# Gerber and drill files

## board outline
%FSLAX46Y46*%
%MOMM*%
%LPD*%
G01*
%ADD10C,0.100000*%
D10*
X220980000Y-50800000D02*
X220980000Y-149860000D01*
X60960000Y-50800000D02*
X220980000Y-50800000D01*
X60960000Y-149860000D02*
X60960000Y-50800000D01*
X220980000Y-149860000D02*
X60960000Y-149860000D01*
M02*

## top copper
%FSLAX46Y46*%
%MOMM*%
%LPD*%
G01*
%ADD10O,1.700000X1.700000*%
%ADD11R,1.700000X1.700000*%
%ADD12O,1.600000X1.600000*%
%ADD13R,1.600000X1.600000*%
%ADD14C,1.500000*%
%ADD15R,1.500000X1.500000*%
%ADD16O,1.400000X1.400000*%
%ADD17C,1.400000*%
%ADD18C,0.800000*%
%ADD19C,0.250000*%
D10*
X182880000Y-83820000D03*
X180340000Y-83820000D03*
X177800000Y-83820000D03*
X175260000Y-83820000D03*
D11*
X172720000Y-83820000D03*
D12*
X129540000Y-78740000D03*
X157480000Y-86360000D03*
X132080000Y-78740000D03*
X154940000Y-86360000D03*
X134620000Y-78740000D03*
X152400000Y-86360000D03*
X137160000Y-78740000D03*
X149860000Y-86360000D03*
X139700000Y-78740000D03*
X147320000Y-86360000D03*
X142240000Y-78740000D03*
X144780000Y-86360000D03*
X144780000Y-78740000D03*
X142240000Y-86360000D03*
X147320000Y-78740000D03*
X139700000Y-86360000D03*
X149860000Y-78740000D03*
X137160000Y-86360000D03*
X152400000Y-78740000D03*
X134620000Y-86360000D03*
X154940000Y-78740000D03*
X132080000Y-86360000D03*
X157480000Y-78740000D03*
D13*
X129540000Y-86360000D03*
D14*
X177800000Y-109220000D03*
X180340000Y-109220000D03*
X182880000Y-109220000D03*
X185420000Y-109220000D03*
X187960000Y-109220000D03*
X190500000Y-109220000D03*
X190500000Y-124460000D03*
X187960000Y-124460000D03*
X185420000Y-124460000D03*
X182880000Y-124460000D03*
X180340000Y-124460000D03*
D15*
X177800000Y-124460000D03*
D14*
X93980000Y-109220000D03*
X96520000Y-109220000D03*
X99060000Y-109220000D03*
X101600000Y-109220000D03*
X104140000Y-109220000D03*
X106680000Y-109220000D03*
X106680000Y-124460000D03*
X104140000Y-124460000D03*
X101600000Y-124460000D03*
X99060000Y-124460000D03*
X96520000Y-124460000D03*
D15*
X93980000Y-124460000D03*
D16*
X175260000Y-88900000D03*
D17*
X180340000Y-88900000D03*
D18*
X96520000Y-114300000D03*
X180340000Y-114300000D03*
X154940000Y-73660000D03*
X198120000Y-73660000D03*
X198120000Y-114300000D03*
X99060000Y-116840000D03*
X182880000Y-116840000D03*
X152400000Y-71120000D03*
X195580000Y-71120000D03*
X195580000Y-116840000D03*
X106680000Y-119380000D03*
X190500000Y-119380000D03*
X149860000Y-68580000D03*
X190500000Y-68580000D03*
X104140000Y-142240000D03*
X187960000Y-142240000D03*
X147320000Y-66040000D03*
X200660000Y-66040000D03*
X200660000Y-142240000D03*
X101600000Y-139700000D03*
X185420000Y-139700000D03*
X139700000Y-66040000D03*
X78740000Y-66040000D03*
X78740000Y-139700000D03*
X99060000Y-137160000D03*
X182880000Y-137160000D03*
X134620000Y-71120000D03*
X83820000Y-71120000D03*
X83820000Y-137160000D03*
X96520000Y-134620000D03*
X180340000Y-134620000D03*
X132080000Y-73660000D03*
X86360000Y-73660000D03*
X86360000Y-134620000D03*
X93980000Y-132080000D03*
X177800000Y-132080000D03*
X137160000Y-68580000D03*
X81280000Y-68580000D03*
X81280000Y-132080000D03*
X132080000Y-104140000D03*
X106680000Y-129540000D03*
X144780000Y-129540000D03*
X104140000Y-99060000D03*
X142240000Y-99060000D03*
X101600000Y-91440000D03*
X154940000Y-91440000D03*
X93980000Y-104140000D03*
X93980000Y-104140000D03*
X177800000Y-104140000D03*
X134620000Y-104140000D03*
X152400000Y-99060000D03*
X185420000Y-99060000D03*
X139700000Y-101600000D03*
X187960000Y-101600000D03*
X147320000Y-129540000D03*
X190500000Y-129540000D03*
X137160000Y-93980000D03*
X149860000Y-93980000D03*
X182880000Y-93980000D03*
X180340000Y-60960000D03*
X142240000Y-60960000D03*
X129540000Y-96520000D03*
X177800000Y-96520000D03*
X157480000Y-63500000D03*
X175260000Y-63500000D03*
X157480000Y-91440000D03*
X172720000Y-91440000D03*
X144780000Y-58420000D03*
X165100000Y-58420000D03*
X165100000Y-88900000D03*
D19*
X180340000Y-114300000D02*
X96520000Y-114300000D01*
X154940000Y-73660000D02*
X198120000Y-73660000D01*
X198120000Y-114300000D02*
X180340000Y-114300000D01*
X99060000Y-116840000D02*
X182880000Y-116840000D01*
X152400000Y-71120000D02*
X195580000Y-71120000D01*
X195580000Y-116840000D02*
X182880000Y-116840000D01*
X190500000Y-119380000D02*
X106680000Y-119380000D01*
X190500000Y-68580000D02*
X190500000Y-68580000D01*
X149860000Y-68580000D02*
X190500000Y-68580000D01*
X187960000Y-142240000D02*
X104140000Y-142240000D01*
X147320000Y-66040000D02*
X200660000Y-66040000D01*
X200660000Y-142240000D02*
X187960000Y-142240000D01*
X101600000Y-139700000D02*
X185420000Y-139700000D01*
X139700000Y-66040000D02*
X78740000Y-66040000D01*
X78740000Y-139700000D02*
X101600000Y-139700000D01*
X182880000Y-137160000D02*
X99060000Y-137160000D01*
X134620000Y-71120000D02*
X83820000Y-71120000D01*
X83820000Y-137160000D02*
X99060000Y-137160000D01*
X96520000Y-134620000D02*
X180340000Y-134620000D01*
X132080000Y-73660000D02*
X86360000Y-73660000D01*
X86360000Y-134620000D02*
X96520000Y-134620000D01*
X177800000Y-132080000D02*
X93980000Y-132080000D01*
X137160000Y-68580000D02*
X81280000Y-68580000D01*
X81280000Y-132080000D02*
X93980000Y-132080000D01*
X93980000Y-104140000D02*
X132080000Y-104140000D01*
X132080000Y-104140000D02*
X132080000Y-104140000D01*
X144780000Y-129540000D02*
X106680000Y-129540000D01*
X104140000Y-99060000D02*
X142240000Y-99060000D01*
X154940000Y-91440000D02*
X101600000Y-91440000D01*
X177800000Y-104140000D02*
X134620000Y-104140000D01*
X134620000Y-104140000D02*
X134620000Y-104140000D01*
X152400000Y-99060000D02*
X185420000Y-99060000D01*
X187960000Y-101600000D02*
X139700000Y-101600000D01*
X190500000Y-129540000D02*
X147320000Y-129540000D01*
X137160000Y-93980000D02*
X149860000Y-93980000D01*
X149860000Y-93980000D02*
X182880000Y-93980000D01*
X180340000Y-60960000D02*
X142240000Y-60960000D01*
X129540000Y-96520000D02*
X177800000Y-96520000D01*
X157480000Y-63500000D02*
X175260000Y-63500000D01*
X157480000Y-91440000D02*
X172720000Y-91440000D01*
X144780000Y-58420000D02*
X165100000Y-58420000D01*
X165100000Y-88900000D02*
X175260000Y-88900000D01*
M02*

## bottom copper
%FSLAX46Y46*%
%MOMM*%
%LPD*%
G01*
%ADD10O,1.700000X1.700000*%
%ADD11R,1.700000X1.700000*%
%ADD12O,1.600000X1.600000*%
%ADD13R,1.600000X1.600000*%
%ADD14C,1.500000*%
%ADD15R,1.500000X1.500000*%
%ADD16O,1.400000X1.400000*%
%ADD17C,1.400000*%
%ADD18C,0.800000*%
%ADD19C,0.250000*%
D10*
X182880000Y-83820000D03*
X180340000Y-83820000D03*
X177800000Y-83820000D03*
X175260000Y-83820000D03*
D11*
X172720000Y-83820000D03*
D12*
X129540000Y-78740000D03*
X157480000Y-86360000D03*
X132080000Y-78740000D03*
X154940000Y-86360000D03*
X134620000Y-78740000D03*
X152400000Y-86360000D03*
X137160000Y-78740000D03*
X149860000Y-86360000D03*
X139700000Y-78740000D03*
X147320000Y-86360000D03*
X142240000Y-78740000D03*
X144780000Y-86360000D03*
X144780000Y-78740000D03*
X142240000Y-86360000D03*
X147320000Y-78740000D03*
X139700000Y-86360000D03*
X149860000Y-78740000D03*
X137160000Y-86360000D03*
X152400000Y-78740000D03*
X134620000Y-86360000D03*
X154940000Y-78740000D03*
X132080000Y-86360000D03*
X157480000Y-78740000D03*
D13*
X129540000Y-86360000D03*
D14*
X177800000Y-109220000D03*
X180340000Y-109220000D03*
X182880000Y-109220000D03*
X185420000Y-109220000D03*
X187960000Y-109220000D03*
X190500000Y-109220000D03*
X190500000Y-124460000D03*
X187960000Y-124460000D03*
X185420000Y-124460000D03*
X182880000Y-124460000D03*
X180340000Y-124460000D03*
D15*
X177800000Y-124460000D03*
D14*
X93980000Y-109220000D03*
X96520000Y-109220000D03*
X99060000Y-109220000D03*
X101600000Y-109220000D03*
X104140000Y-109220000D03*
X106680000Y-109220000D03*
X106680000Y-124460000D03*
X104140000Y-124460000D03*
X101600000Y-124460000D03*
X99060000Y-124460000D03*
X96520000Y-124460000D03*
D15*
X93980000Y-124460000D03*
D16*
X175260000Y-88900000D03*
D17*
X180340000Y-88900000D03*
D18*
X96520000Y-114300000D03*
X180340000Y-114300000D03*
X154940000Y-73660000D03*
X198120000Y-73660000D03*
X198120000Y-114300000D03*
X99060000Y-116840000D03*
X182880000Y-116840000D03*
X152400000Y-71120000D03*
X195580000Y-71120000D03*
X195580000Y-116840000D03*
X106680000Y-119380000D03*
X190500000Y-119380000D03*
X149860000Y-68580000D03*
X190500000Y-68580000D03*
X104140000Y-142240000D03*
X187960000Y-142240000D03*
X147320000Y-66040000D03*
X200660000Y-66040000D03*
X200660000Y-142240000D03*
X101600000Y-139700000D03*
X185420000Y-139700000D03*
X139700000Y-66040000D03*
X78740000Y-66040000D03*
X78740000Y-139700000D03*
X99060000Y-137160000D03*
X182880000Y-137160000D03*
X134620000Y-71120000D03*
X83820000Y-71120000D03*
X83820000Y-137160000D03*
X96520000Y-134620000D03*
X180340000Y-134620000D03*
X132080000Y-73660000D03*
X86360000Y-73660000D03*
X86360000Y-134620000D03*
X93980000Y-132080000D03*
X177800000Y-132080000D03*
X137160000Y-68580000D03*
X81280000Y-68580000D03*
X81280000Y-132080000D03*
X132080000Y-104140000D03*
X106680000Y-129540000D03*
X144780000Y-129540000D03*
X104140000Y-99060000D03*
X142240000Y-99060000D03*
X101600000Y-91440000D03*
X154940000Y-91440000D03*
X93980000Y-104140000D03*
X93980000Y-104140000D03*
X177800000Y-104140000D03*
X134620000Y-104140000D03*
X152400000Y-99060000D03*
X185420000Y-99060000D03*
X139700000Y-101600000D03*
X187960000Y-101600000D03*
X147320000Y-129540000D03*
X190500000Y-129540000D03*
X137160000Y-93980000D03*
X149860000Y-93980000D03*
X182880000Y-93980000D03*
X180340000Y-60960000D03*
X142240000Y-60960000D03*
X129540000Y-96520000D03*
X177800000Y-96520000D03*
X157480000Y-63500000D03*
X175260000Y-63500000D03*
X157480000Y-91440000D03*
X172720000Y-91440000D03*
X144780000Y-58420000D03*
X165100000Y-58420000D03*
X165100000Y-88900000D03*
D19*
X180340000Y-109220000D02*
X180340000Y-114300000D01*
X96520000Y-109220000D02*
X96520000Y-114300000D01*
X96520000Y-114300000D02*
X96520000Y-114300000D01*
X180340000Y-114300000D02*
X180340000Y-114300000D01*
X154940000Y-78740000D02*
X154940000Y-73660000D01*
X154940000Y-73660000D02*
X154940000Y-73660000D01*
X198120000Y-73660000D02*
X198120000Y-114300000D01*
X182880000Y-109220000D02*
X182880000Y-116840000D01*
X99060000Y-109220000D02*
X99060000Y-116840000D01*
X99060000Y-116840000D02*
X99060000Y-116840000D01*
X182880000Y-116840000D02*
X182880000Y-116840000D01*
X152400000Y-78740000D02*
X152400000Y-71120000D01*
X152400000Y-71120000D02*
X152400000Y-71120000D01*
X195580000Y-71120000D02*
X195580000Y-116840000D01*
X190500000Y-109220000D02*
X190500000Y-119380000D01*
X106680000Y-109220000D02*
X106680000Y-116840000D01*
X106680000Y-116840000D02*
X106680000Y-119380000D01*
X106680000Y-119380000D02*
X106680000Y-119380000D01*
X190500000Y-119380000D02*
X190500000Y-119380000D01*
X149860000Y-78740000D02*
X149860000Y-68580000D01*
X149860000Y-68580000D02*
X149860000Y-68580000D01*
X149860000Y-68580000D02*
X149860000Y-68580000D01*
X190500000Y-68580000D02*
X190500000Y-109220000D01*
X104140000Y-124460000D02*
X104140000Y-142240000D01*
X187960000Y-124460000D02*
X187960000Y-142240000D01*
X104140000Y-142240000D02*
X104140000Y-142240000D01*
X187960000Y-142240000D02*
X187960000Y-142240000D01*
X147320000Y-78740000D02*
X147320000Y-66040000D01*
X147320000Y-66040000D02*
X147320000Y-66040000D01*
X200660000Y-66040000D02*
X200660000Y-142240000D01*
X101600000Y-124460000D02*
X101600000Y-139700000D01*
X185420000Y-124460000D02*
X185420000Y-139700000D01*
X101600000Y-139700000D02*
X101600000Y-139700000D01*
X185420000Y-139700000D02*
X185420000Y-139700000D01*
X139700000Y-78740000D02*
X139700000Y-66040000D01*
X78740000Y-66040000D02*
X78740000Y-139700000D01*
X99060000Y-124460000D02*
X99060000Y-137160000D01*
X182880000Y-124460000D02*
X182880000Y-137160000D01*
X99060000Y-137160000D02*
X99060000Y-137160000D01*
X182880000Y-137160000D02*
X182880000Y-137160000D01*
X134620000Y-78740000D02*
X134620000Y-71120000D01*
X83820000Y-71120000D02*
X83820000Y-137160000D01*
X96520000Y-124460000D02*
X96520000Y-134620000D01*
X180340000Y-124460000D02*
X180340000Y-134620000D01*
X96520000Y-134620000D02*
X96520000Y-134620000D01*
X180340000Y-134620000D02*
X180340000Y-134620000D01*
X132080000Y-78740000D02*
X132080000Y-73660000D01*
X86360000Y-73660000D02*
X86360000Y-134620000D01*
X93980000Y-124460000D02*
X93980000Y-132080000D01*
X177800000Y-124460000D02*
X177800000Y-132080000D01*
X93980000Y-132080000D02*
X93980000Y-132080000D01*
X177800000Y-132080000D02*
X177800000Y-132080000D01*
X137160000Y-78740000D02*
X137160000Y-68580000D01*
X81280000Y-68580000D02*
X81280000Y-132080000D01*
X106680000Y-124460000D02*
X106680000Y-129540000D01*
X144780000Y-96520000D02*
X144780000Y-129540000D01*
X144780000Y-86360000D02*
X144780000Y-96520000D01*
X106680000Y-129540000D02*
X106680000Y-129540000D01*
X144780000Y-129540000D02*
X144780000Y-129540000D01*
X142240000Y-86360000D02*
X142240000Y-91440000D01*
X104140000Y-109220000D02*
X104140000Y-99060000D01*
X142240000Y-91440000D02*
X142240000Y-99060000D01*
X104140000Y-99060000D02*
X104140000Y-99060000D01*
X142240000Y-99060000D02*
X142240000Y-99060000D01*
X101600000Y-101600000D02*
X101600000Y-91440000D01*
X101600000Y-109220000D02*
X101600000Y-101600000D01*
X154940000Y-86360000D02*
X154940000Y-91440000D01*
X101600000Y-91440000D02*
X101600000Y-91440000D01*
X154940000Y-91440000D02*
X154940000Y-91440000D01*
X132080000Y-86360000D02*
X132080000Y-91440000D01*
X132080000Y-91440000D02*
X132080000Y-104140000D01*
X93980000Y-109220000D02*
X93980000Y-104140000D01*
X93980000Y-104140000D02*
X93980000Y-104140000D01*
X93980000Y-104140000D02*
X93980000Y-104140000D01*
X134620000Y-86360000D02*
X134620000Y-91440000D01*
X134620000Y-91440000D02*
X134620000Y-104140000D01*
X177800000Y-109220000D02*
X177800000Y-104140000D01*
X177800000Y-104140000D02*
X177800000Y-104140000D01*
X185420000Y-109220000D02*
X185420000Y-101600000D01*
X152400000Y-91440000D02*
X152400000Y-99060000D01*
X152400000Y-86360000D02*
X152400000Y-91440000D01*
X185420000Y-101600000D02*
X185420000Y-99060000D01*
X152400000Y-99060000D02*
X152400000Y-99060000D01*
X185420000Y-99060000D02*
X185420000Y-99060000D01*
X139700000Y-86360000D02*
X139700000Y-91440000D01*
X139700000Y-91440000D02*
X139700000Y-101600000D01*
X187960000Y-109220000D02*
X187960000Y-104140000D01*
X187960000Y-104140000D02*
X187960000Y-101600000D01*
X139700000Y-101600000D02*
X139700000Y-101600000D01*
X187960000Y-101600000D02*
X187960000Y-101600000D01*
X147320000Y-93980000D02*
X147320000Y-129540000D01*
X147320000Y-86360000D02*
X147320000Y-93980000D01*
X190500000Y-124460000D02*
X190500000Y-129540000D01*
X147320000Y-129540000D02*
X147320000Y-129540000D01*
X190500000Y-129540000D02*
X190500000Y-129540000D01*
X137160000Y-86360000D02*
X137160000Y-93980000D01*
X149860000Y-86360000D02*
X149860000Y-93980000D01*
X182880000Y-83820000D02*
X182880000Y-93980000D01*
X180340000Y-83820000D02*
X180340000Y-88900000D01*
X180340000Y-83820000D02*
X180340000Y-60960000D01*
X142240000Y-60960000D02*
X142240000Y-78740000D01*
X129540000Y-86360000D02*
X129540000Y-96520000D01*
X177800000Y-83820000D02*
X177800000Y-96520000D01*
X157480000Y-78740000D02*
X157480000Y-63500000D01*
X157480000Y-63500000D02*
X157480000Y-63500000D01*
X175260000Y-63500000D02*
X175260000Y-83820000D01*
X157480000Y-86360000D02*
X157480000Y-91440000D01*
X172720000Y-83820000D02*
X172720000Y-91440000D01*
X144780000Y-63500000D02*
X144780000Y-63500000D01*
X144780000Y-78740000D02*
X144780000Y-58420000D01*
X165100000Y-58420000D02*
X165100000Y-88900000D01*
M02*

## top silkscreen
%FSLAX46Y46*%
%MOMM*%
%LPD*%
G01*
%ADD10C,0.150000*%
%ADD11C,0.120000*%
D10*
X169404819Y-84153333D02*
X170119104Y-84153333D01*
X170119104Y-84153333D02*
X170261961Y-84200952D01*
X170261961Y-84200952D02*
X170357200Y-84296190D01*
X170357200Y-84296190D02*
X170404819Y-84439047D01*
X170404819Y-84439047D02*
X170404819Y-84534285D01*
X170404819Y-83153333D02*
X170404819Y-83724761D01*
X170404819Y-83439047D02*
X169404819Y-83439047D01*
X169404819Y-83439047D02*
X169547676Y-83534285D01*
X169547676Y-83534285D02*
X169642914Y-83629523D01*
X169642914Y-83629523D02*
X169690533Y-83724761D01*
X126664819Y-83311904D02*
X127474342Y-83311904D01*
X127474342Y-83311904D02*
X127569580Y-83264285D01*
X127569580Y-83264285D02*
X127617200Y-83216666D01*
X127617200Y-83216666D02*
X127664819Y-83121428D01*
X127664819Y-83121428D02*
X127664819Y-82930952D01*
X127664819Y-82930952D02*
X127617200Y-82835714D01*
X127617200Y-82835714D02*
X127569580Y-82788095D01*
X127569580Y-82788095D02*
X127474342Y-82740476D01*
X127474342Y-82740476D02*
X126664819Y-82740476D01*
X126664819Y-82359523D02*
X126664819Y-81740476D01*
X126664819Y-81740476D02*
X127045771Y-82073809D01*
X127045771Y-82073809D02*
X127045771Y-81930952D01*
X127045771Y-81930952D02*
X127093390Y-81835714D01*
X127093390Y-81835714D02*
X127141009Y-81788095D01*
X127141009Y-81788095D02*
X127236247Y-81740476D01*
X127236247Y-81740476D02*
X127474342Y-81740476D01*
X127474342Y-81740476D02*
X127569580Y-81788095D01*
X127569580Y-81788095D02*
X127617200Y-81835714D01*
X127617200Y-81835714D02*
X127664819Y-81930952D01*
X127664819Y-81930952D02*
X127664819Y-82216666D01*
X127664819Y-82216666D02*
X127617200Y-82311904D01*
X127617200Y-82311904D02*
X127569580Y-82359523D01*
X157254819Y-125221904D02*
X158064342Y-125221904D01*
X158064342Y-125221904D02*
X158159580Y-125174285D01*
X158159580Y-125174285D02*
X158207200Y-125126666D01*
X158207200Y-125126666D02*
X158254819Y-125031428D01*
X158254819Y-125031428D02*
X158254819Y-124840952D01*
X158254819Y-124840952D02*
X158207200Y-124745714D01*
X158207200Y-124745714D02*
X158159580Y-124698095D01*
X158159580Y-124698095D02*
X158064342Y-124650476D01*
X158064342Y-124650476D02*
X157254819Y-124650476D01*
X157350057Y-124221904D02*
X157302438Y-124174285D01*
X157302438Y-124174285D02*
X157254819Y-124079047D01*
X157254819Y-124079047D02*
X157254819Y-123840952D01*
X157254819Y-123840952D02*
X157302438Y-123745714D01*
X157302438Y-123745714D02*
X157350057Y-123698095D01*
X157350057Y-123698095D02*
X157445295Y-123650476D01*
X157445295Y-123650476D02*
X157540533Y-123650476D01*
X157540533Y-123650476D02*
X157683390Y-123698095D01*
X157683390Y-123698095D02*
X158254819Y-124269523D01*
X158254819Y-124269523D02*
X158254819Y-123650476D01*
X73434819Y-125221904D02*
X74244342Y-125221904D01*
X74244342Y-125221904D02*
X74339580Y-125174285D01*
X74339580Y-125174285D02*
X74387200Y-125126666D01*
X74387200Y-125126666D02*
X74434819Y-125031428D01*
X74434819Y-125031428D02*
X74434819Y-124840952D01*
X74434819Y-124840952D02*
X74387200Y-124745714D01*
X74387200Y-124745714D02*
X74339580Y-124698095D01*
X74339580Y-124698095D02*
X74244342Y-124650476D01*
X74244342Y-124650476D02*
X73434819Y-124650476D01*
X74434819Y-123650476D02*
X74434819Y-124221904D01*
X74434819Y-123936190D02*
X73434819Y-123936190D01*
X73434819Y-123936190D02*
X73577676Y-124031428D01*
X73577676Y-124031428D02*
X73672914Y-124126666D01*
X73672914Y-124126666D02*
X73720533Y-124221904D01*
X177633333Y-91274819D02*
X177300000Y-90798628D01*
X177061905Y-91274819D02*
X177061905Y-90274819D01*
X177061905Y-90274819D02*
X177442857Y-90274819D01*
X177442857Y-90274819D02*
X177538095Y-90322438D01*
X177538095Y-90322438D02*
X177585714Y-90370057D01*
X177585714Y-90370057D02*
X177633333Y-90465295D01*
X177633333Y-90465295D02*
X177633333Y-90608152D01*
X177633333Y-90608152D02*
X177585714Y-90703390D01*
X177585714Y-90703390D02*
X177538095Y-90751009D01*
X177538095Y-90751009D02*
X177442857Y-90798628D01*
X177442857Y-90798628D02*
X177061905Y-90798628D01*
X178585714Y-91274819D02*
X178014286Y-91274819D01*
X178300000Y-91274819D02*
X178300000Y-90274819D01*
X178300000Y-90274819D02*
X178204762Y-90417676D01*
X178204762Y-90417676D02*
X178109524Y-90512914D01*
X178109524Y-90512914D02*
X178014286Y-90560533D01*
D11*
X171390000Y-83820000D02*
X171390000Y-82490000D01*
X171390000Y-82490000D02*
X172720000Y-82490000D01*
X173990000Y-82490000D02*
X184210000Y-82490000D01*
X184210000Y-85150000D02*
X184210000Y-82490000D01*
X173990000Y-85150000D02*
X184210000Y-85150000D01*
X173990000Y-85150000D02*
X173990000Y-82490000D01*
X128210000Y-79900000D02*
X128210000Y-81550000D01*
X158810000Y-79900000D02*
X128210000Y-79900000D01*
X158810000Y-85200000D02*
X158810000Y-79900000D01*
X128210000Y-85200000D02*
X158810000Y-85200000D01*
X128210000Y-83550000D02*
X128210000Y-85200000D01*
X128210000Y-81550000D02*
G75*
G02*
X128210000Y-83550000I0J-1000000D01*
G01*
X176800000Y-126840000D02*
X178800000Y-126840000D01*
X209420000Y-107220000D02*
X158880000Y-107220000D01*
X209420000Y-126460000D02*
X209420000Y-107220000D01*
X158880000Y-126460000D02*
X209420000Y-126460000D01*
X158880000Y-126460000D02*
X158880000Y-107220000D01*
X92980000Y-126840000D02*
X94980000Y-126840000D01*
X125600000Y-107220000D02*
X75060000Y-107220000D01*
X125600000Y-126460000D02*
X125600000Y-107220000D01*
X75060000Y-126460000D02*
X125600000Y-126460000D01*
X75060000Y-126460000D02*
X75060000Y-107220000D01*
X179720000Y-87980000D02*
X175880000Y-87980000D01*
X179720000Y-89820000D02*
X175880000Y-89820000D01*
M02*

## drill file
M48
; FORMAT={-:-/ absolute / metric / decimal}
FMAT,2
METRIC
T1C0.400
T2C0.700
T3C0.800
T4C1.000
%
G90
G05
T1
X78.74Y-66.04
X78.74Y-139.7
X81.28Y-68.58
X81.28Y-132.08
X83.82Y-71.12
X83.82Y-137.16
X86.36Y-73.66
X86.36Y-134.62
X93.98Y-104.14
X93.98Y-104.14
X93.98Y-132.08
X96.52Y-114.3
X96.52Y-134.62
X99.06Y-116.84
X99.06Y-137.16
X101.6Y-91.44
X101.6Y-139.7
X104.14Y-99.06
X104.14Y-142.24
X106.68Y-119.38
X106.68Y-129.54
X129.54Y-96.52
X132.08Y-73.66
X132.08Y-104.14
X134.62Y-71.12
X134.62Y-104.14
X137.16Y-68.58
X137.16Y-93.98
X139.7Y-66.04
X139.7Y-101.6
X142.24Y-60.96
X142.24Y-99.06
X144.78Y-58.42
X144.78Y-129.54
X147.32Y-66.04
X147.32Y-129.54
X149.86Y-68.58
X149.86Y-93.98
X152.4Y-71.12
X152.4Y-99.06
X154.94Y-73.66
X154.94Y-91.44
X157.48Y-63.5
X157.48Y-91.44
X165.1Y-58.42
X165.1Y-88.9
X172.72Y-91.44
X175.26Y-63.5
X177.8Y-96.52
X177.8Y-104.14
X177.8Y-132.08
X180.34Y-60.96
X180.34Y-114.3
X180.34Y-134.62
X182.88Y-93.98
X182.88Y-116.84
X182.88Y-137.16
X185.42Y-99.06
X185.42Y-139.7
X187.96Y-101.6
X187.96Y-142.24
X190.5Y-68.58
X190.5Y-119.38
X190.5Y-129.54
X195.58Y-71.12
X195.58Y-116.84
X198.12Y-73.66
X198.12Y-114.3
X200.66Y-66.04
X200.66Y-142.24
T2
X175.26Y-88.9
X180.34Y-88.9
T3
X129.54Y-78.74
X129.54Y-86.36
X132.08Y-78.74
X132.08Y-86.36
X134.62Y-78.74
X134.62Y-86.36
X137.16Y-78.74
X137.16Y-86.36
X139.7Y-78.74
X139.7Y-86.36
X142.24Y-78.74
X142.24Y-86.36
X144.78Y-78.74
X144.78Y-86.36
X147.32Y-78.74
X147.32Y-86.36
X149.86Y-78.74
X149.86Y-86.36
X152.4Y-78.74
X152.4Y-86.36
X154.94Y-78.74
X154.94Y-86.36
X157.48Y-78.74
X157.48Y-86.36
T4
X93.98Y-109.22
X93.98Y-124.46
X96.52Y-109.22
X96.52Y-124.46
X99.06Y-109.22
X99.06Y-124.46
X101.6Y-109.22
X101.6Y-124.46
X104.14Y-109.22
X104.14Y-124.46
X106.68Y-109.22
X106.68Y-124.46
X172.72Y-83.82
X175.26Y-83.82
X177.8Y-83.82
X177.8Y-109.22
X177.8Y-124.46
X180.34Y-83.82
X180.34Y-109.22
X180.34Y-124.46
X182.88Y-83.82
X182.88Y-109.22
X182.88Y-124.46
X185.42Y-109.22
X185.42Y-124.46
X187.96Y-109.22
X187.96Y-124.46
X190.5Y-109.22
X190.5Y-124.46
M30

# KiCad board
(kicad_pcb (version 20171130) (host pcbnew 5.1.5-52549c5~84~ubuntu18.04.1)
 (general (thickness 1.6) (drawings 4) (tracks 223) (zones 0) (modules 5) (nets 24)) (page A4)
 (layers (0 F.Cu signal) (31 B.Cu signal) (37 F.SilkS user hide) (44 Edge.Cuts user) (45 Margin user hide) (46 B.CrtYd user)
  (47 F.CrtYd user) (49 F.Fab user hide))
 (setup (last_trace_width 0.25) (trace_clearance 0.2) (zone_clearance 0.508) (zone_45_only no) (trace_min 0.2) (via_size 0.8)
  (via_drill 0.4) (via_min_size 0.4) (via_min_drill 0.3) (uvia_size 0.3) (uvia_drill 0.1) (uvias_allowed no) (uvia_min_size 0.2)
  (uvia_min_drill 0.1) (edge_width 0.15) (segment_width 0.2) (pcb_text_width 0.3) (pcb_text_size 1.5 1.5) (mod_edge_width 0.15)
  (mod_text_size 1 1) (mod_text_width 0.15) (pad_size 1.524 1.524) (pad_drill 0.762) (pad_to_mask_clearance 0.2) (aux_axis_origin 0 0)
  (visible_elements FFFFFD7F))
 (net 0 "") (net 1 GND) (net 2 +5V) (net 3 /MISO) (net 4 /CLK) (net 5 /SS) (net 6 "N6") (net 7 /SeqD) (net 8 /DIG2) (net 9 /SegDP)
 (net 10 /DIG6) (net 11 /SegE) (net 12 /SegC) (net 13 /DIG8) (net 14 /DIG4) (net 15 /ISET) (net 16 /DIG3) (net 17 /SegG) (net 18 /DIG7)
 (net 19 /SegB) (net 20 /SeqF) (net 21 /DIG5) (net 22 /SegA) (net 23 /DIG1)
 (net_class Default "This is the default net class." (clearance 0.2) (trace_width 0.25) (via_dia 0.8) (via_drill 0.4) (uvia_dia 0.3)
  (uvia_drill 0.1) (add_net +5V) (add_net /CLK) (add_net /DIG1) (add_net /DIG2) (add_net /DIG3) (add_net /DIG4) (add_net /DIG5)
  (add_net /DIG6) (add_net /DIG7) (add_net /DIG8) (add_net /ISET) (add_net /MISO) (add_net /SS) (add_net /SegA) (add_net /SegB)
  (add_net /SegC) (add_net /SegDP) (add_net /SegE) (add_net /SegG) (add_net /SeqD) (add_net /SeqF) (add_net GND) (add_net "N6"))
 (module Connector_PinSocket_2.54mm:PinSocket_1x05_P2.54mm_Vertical (layer F.Cu) (at 172.72 83.82 90)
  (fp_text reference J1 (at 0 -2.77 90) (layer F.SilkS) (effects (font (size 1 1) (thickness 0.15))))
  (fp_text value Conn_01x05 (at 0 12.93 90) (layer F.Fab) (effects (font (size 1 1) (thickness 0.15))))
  (fp_line (start 0 -1.33) (end 1.33 -1.33) (layer F.SilkS) (width 0.12))
  (fp_line (start 1.33 -1.33) (end 1.33 0) (layer F.SilkS) (width 0.12))
  (fp_line (start 1.33 1.27) (end 1.33 11.49) (layer F.SilkS) (width 0.12))
  (fp_line (start -1.33 11.49) (end 1.33 11.49) (layer F.SilkS) (width 0.12))
  (fp_line (start -1.33 1.27) (end -1.33 11.49) (layer F.SilkS) (width 0.12))
  (fp_line (start -1.33 1.27) (end 1.33 1.27) (layer F.SilkS) (width 0.12))
  (pad 5 thru_hole oval (at 0 10.16 90) (size 1.7 1.7) (drill 1) (layers *.Cu *.Mask) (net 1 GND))
  (pad 4 thru_hole oval (at 0 7.62 90) (size 1.7 1.7) (drill 1) (layers *.Cu *.Mask) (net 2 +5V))
  (pad 3 thru_hole oval (at 0 5.08 90) (size 1.7 1.7) (drill 1) (layers *.Cu *.Mask) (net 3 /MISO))
  (pad 2 thru_hole oval (at 0 2.54 90) (size 1.7 1.7) (drill 1) (layers *.Cu *.Mask) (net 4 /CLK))
  (pad 1 thru_hole rect (at 0 0 90) (size 1.7 1.7) (drill 1) (layers *.Cu *.Mask) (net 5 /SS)))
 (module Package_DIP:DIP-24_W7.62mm (layer F.Cu) (at 129.54 86.36 90)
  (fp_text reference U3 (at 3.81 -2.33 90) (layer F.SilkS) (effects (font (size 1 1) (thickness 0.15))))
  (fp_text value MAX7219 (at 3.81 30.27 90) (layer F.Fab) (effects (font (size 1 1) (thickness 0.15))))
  (fp_line (start 6.46 -1.33) (end 4.81 -1.33) (layer F.SilkS) (width 0.12))
  (fp_line (start 6.46 29.27) (end 6.46 -1.33) (layer F.SilkS) (width 0.12))
  (fp_line (start 1.16 29.27) (end 6.46 29.27) (layer F.SilkS) (width 0.12))
  (fp_line (start 1.16 -1.33) (end 1.16 29.27) (layer F.SilkS) (width 0.12))
  (fp_line (start 2.81 -1.33) (end 1.16 -1.33) (layer F.SilkS) (width 0.12))
  (fp_arc (start 3.81 -1.33) (end 2.81 -1.33) (angle -180) (layer F.SilkS) (width 0.12))
  (pad 24 thru_hole oval (at 7.62 0 90) (size 1.6 1.6) (drill 0.8) (layers *.Cu *.Mask) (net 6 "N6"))
  (pad 12 thru_hole oval (at 0 27.94 90) (size 1.6 1.6) (drill 0.8) (layers *.Cu *.Mask) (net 5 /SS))
  (pad 23 thru_hole oval (at 7.62 2.54 90) (size 1.6 1.6) (drill 0.8) (layers *.Cu *.Mask) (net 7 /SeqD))
  (pad 11 thru_hole oval (at 0 25.4 90) (size 1.6 1.6) (drill 0.8) (layers *.Cu *.Mask) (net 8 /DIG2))
  (pad 22 thru_hole oval (at 7.62 5.08 90) (size 1.6 1.6) (drill 0.8) (layers *.Cu *.Mask) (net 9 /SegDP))
  (pad 10 thru_hole oval (at 0 22.86 90) (size 1.6 1.6) (drill 0.8) (layers *.Cu *.Mask) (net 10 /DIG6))
  (pad 21 thru_hole oval (at 7.62 7.62 90) (size 1.6 1.6) (drill 0.8) (layers *.Cu *.Mask) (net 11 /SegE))
  (pad 9 thru_hole oval (at 0 20.32 90) (size 1.6 1.6) (drill 0.8) (layers *.Cu *.Mask) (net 1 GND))
  (pad 20 thru_hole oval (at 7.62 10.16 90) (size 1.6 1.6) (drill 0.8) (layers *.Cu *.Mask) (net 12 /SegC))
  (pad 8 thru_hole oval (at 0 17.78 90) (size 1.6 1.6) (drill 0.8) (layers *.Cu *.Mask) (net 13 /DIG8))
  (pad 19 thru_hole oval (at 7.62 12.7 90) (size 1.6 1.6) (drill 0.8) (layers *.Cu *.Mask) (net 2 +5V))
  (pad 7 thru_hole oval (at 0 15.24 90) (size 1.6 1.6) (drill 0.8) (layers *.Cu *.Mask) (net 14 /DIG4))
  (pad 18 thru_hole oval (at 7.62 15.24 90) (size 1.6 1.6) (drill 0.8) (layers *.Cu *.Mask) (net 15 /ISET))
  (pad 6 thru_hole oval (at 0 12.7 90) (size 1.6 1.6) (drill 0.8) (layers *.Cu *.Mask) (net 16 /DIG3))
  (pad 17 thru_hole oval (at 7.62 17.78 90) (size 1.6 1.6) (drill 0.8) (layers *.Cu *.Mask) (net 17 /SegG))
  (pad 5 thru_hole oval (at 0 10.16 90) (size 1.6 1.6) (drill 0.8) (layers *.Cu *.Mask) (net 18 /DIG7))
  (pad 16 thru_hole oval (at 7.62 20.32 90) (size 1.6 1.6) (drill 0.8) (layers *.Cu *.Mask) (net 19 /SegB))
  (pad 4 thru_hole oval (at 0 7.62 90) (size 1.6 1.6) (drill 0.8) (layers *.Cu *.Mask) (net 1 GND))
  (pad 15 thru_hole oval (at 7.62 22.86 90) (size 1.6 1.6) (drill 0.8) (layers *.Cu *.Mask) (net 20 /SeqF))
  (pad 3 thru_hole oval (at 0 5.08 90) (size 1.6 1.6) (drill 0.8) (layers *.Cu *.Mask) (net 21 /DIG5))
  (pad 14 thru_hole oval (at 7.62 25.4 90) (size 1.6 1.6) (drill 0.8) (layers *.Cu *.Mask) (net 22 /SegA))
  (pad 2 thru_hole oval (at 0 2.54 90) (size 1.6 1.6) (drill 0.8) (layers *.Cu *.Mask) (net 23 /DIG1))
  (pad 13 thru_hole oval (at 7.62 27.94 90) (size 1.6 1.6) (drill 0.8) (layers *.Cu *.Mask) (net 4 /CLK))
  (pad 1 thru_hole rect (at 0 0 90) (size 1.6 1.6) (drill 0.8) (layers *.Cu *.Mask) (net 3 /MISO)))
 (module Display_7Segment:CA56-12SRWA (layer F.Cu) (at 177.8 124.46 90)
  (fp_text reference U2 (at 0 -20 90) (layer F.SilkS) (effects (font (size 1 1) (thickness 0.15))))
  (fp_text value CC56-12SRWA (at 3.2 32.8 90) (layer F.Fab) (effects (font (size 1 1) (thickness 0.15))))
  (fp_line (start -2.38 -1) (end -2.38 1) (layer F.SilkS) (width 0.12))
  (fp_line (start 17.24 31.62) (end 17.24 -18.92) (layer F.SilkS) (width 0.12))
  (fp_line (start -2 31.62) (end 17.24 31.62) (layer F.SilkS) (width 0.12))
  (fp_line (start -2 -18.92) (end -2 31.62) (layer F.SilkS) (width 0.12))
  (fp_line (start -2 -18.92) (end 17.24 -18.92) (layer F.SilkS) (width 0.12))
  (pad 12 thru_hole circle (at 15.24 0 90) (size 1.5 1.5) (drill 1) (layers *.Cu *.Mask) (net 21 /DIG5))
  (pad 11 thru_hole circle (at 15.24 2.54 90) (size 1.5 1.5) (drill 1) (layers *.Cu *.Mask) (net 22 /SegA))
  (pad 10 thru_hole circle (at 15.24 5.08 90) (size 1.5 1.5) (drill 1) (layers *.Cu *.Mask) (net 20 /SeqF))
  (pad 9 thru_hole circle (at 15.24 7.62 90) (size 1.5 1.5) (drill 1) (layers *.Cu *.Mask) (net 10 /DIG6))
  (pad 8 thru_hole circle (at 15.24 10.16 90) (size 1.5 1.5) (drill 1) (layers *.Cu *.Mask) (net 18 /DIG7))
  (pad 7 thru_hole circle (at 15.24 12.7 90) (size 1.5 1.5) (drill 1) (layers *.Cu *.Mask) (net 19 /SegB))
  (pad 6 thru_hole circle (at 0 12.7 90) (size 1.5 1.5) (drill 1) (layers *.Cu *.Mask) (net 13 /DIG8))
  (pad 5 thru_hole circle (at 0 10.16 90) (size 1.5 1.5) (drill 1) (layers *.Cu *.Mask) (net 17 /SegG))
  (pad 4 thru_hole circle (at 0 7.62 90) (size 1.5 1.5) (drill 1) (layers *.Cu *.Mask) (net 12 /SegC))
  (pad 3 thru_hole circle (at 0 5.08 90) (size 1.5 1.5) (drill 1) (layers *.Cu *.Mask) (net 9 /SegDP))
  (pad 2 thru_hole circle (at 0 2.54 90) (size 1.5 1.5) (drill 1) (layers *.Cu *.Mask) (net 7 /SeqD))
  (pad 1 thru_hole rect (at 0 0 90) (size 1.5 1.5) (drill 1) (layers *.Cu *.Mask) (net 11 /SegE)))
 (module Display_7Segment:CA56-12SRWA (layer F.Cu) (at 93.98 124.46 90)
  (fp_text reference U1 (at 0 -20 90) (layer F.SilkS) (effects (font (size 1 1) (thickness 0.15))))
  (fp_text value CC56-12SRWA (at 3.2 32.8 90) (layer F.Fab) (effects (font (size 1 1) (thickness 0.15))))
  (fp_line (start -2.38 -1) (end -2.38 1) (layer F.SilkS) (width 0.12))
  (fp_line (start 17.24 31.62) (end 17.24 -18.92) (layer F.SilkS) (width 0.12))
  (fp_line (start -2 31.62) (end 17.24 31.62) (layer F.SilkS) (width 0.12))
  (fp_line (start -2 -18.92) (end -2 31.62) (layer F.SilkS) (width 0.12))
  (fp_line (start -2 -18.92) (end 17.24 -18.92) (layer F.SilkS) (width 0.12))
  (pad 12 thru_hole circle (at 15.24 0 90) (size 1.5 1.5) (drill 1) (layers *.Cu *.Mask) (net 23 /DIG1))
  (pad 11 thru_hole circle (at 15.24 2.54 90) (size 1.5 1.5) (drill 1) (layers *.Cu *.Mask) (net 22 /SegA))
  (pad 10 thru_hole circle (at 15.24 5.08 90) (size 1.5 1.5) (drill 1) (layers *.Cu *.Mask) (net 20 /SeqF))
  (pad 9 thru_hole circle (at 15.24 7.62 90) (size 1.5 1.5) (drill 1) (layers *.Cu *.Mask) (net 8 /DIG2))
  (pad 8 thru_hole circle (at 15.24 10.16 90) (size 1.5 1.5) (drill 1) (layers *.Cu *.Mask) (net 16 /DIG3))
  (pad 7 thru_hole circle (at 15.24 12.7 90) (size 1.5 1.5) (drill 1) (layers *.Cu *.Mask) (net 19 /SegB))
  (pad 6 thru_hole circle (at 0 12.7 90) (size 1.5 1.5) (drill 1) (layers *.Cu *.Mask) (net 14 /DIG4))
  (pad 5 thru_hole circle (at 0 10.16 90) (size 1.5 1.5) (drill 1) (layers *.Cu *.Mask) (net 17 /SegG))
  (pad 4 thru_hole circle (at 0 7.62 90) (size 1.5 1.5) (drill 1) (layers *.Cu *.Mask) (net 12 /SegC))
  (pad 3 thru_hole circle (at 0 5.08 90) (size 1.5 1.5) (drill 1) (layers *.Cu *.Mask) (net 9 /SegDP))
  (pad 2 thru_hole circle (at 0 2.54 90) (size 1.5 1.5) (drill 1) (layers *.Cu *.Mask) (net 7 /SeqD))
  (pad 1 thru_hole rect (at 0 0 90) (size 1.5 1.5) (drill 1) (layers *.Cu *.Mask) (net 11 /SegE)))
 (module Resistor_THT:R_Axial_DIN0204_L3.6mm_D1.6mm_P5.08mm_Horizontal (layer F.Cu) (at 180.34 88.9 180)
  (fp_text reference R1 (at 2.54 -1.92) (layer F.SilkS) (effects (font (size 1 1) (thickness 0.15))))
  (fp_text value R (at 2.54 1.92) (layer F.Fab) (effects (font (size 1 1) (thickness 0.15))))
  (fp_line (start 0.62 0.92) (end 4.46 0.92) (layer F.SilkS) (width 0.12))
  (fp_line (start 0.62 -0.92) (end 4.46 -0.92) (layer F.SilkS) (width 0.12))
  (pad 2 thru_hole oval (at 5.08 0 180) (size 1.4 1.4) (drill 0.7) (layers *.Cu *.Mask) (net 15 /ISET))
  (pad 1 thru_hole circle (at 0 0 180) (size 1.4 1.4) (drill 0.7) (layers *.Cu *.Mask) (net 2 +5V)))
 (gr_line (start 220.98 50.8) (end 220.98 149.86) (layer Edge.Cuts) (width 0.1))
 (gr_line (start 60.96 50.8) (end 220.98 50.8) (layer Edge.Cuts) (width 0.1))
 (gr_line (start 60.96 149.86) (end 60.96 50.8) (layer Edge.Cuts) (width 0.1))
 (gr_line (start 220.98 149.86) (end 60.96 149.86) (layer Edge.Cuts) (width 0.1))
 (segment (start 180.34 109.22) (end 180.34 114.3) (width 0.25) (layer B.Cu) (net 22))
 (segment (start 96.52 109.22) (end 96.52 114.3) (width 0.25) (layer B.Cu) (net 22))
 (segment (start 96.52 114.3) (end 96.52 114.3) (width 0.25) (layer B.Cu) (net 22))
 (via (at 96.52 114.3) (size 0.8) (drill 0.4) (layers F.Cu B.Cu) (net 22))
 (segment (start 180.34 114.3) (end 180.34 114.3) (width 0.25) (layer B.Cu) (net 22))
 (via (at 180.34 114.3) (size 0.8) (drill 0.4) (layers F.Cu B.Cu) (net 22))
 (segment (start 180.34 114.3) (end 96.52 114.3) (width 0.25) (layer F.Cu) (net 22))
 (segment (start 154.94 78.74) (end 154.94 73.66) (width 0.25) (layer B.Cu) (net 22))
 (segment (start 154.94 73.66) (end 154.94 73.66) (width 0.25) (layer B.Cu) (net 22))
 (via (at 154.94 73.66) (size 0.8) (drill 0.4) (layers F.Cu B.Cu) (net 22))
 (via (at 198.12 73.66) (size 0.8) (drill 0.4) (layers F.Cu B.Cu) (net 22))
 (segment (start 154.94 73.66) (end 198.12 73.66) (width 0.25) (layer F.Cu) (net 22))
 (segment (start 198.12 73.66) (end 198.12 114.3) (width 0.25) (layer B.Cu) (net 22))
 (via (at 198.12 114.3) (size 0.8) (drill 0.4) (layers F.Cu B.Cu) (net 22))
 (segment (start 198.12 114.3) (end 180.34 114.3) (width 0.25) (layer F.Cu) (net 22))
 (segment (start 182.88 109.22) (end 182.88 116.84) (width 0.25) (layer B.Cu) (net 20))
 (segment (start 99.06 109.22) (end 99.06 116.84) (width 0.25) (layer B.Cu) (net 20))
 (segment (start 99.06 116.84) (end 99.06 116.84) (width 0.25) (layer B.Cu) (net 20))
 (via (at 99.06 116.84) (size 0.8) (drill 0.4) (layers F.Cu B.Cu) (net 20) (status 1000000))
 (segment (start 182.88 116.84) (end 182.88 116.84) (width 0.25) (layer B.Cu) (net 20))
 (via (at 182.88 116.84) (size 0.8) (drill 0.4) (layers F.Cu B.Cu) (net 20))
 (segment (start 99.06 116.84) (end 182.88 116.84) (width 0.25) (layer F.Cu) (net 20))
 (segment (start 152.4 78.74) (end 152.4 71.12) (width 0.25) (layer B.Cu) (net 20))
 (segment (start 152.4 71.12) (end 152.4 71.12) (width 0.25) (layer B.Cu) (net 20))
 (via (at 152.4 71.12) (size 0.8) (drill 0.4) (layers F.Cu B.Cu) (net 20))
 (via (at 195.58 71.12) (size 0.8) (drill 0.4) (layers F.Cu B.Cu) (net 20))
 (segment (start 152.4 71.12) (end 195.58 71.12) (width 0.25) (layer F.Cu) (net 20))
 (segment (start 195.58 71.12) (end 195.58 116.84) (width 0.25) (layer B.Cu) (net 20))
 (via (at 195.58 116.84) (size 0.8) (drill 0.4) (layers F.Cu B.Cu) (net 20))
 (segment (start 195.58 116.84) (end 182.88 116.84) (width 0.25) (layer F.Cu) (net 20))
 (segment (start 190.5 109.22) (end 190.5 119.38) (width 0.25) (layer B.Cu) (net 19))
 (segment (start 106.68 109.22) (end 106.68 116.84) (width 0.25) (layer B.Cu) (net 19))
 (segment (start 106.68 116.84) (end 106.68 119.38) (width 0.25) (layer B.Cu) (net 19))
 (segment (start 106.68 119.38) (end 106.68 119.38) (width 0.25) (layer B.Cu) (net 19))
 (via (at 106.68 119.38) (size 0.8) (drill 0.4) (layers F.Cu B.Cu) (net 19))
 (segment (start 190.5 119.38) (end 190.5 119.38) (width 0.25) (layer B.Cu) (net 19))
 (via (at 190.5 119.38) (size 0.8) (drill 0.4) (layers F.Cu B.Cu) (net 19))
 (segment (start 190.5 119.38) (end 106.68 119.38) (width 0.25) (layer F.Cu) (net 19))
 (segment (start 149.86 78.74) (end 149.86 68.58) (width 0.25) (layer B.Cu) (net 19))
 (segment (start 149.86 68.58) (end 149.86 68.58) (width 0.25) (layer B.Cu) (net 19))
 (segment (start 149.86 68.58) (end 149.86 68.58) (width 0.25) (layer B.Cu) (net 19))
 (via (at 149.86 68.58) (size 0.8) (drill 0.4) (layers F.Cu B.Cu) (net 19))
 (segment (start 190.5 68.58) (end 190.5 68.58) (width 0.25) (layer F.Cu) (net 19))
 (segment (start 149.86 68.58) (end 190.5 68.58) (width 0.25) (layer F.Cu) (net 19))
 (via (at 190.5 68.58) (size 0.8) (drill 0.4) (layers F.Cu B.Cu) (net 19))
 (segment (start 190.5 68.58) (end 190.5 109.22) (width 0.25) (layer B.Cu) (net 19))
 (segment (start 104.14 124.46) (end 104.14 142.24) (width 0.25) (layer B.Cu) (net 17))
 (segment (start 187.96 124.46) (end 187.96 142.24) (width 0.25) (layer B.Cu) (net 17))
 (segment (start 104.14 142.24) (end 104.14 142.24) (width 0.25) (layer B.Cu) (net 17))
 (via (at 104.14 142.24) (size 0.8) (drill 0.4) (layers F.Cu B.Cu) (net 17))
 (segment (start 187.96 142.24) (end 187.96 142.24) (width 0.25) (layer B.Cu) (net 17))
 (via (at 187.96 142.24) (size 0.8) (drill 0.4) (layers F.Cu B.Cu) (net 17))
 (segment (start 187.96 142.24) (end 104.14 142.24) (width 0.25) (layer F.Cu) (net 17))
 (segment (start 147.32 78.74) (end 147.32 66.04) (width 0.25) (layer B.Cu) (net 17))
 (segment (start 147.32 66.04) (end 147.32 66.04) (width 0.25) (layer B.Cu) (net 17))
 (via (at 147.32 66.04) (size 0.8) (drill 0.4) (layers F.Cu B.Cu) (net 17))
 (via (at 200.66 66.04) (size 0.8) (drill 0.4) (layers F.Cu B.Cu) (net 17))
 (segment (start 147.32 66.04) (end 200.66 66.04) (width 0.25) (layer F.Cu) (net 17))
 (segment (start 200.66 66.04) (end 200.66 142.24) (width 0.25) (layer B.Cu) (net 17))
 (via (at 200.66 142.24) (size 0.8) (drill 0.4) (layers F.Cu B.Cu) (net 17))
 (segment (start 200.66 142.24) (end 187.96 142.24) (width 0.25) (layer F.Cu) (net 17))
 (segment (start 101.6 124.46) (end 101.6 139.7) (width 0.25) (layer B.Cu) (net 12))
 (segment (start 185.42 124.46) (end 185.42 139.7) (width 0.25) (layer B.Cu) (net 12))
 (segment (start 101.6 139.7) (end 101.6 139.7) (width 0.25) (layer B.Cu) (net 12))
 (via (at 101.6 139.7) (size 0.8) (drill 0.4) (layers F.Cu B.Cu) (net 12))
 (segment (start 185.42 139.7) (end 185.42 139.7) (width 0.25) (layer B.Cu) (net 12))
 (via (at 185.42 139.7) (size 0.8) (drill 0.4) (layers F.Cu B.Cu) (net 12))
 (segment (start 101.6 139.7) (end 185.42 139.7) (width 0.25) (layer F.Cu) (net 12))
 (segment (start 139.7 78.74) (end 139.7 66.04) (width 0.25) (layer B.Cu) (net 12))
 (via (at 139.7 66.04) (size 0.8) (drill 0.4) (layers F.Cu B.Cu) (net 12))
 (via (at 78.74 66.04) (size 0.8) (drill 0.4) (layers F.Cu B.Cu) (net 12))
 (segment (start 139.7 66.04) (end 78.74 66.04) (width 0.25) (layer F.Cu) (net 12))
 (via (at 78.74 139.7) (size 0.8) (drill 0.4) (layers F.Cu B.Cu) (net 12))
 (segment (start 78.74 66.04) (end 78.74 139.7) (width 0.25) (layer B.Cu) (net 12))
 (segment (start 78.74 139.7) (end 101.6 139.7) (width 0.25) (layer F.Cu) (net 12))
 (segment (start 99.06 124.46) (end 99.06 137.16) (width 0.25) (layer B.Cu) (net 9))
 (segment (start 182.88 124.46) (end 182.88 137.16) (width 0.25) (layer B.Cu) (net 9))
 (segment (start 99.06 137.16) (end 99.06 137.16) (width 0.25) (layer B.Cu) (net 9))
 (via (at 99.06 137.16) (size 0.8) (drill 0.4) (layers F.Cu B.Cu) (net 9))
 (segment (start 182.88 137.16) (end 182.88 137.16) (width 0.25) (layer B.Cu) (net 9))
 (via (at 182.88 137.16) (size 0.8) (drill 0.4) (layers F.Cu B.Cu) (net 9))
 (segment (start 182.88 137.16) (end 99.06 137.16) (width 0.25) (layer F.Cu) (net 9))
 (via (at 134.62 71.12) (size 0.8) (drill 0.4) (layers F.Cu B.Cu) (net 9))
 (segment (start 134.62 78.74) (end 134.62 71.12) (width 0.25) (layer B.Cu) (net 9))
 (via (at 83.82 71.12) (size 0.8) (drill 0.4) (layers F.Cu B.Cu) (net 9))
 (segment (start 134.62 71.12) (end 83.82 71.12) (width 0.25) (layer F.Cu) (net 9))
 (via (at 83.82 137.16) (size 0.8) (drill 0.4) (layers F.Cu B.Cu) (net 9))
 (segment (start 83.82 71.12) (end 83.82 137.16) (width 0.25) (layer B.Cu) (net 9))
 (segment (start 83.82 137.16) (end 99.06 137.16) (width 0.25) (layer F.Cu) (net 9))
 (segment (start 96.52 124.46) (end 96.52 134.62) (width 0.25) (layer B.Cu) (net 7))
 (segment (start 180.34 124.46) (end 180.34 134.62) (width 0.25) (layer B.Cu) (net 7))
 (segment (start 96.52 134.62) (end 96.52 134.62) (width 0.25) (layer B.Cu) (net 7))
 (via (at 96.52 134.62) (size 0.8) (drill 0.4) (layers F.Cu B.Cu) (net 7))
 (segment (start 180.34 134.62) (end 180.34 134.62) (width 0.25) (layer B.Cu) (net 7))
 (via (at 180.34 134.62) (size 0.8) (drill 0.4) (layers F.Cu B.Cu) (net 7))
 (segment (start 96.52 134.62) (end 180.34 134.62) (width 0.25) (layer F.Cu) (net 7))
 (segment (start 132.08 78.74) (end 132.08 73.66) (width 0.25) (layer B.Cu) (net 7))
 (via (at 132.08 73.66) (size 0.8) (drill 0.4) (layers F.Cu B.Cu) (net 7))
 (via (at 86.36 73.66) (size 0.8) (drill 0.4) (layers F.Cu B.Cu) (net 7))
 (segment (start 132.08 73.66) (end 86.36 73.66) (width 0.25) (layer F.Cu) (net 7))
 (via (at 86.36 134.62) (size 0.8) (drill 0.4) (layers F.Cu B.Cu) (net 7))
 (segment (start 86.36 73.66) (end 86.36 134.62) (width 0.25) (layer B.Cu) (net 7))
 (segment (start 86.36 134.62) (end 96.52 134.62) (width 0.25) (layer F.Cu) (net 7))
 (segment (start 93.98 124.46) (end 93.98 132.08) (width 0.25) (layer B.Cu) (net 11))
 (segment (start 177.8 124.46) (end 177.8 132.08) (width 0.25) (layer B.Cu) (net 11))
 (segment (start 93.98 132.08) (end 93.98 132.08) (width 0.25) (layer B.Cu) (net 11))
 (via (at 93.98 132.08) (size 0.8) (drill 0.4) (layers F.Cu B.Cu) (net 11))
 (segment (start 177.8 132.08) (end 177.8 132.08) (width 0.25) (layer B.Cu) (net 11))
 (via (at 177.8 132.08) (size 0.8) (drill 0.4) (layers F.Cu B.Cu) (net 11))
 (segment (start 177.8 132.08) (end 93.98 132.08) (width 0.25) (layer F.Cu) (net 11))
 (segment (start 137.16 78.74) (end 137.16 68.58) (width 0.25) (layer B.Cu) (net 11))
 (via (at 137.16 68.58) (size 0.8) (drill 0.4) (layers F.Cu B.Cu) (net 11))
 (via (at 81.28 68.58) (size 0.8) (drill 0.4) (layers F.Cu B.Cu) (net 11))
 (segment (start 137.16 68.58) (end 81.28 68.58) (width 0.25) (layer F.Cu) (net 11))
 (via (at 81.28 132.08) (size 0.8) (drill 0.4) (layers F.Cu B.Cu) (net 11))
 (segment (start 81.28 68.58) (end 81.28 132.08) (width 0.25) (layer B.Cu) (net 11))
 (segment (start 81.28 132.08) (end 93.98 132.08) (width 0.25) (layer F.Cu) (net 11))
 (segment (start 93.98 104.14) (end 132.08 104.14) (width 0.25) (layer F.Cu) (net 23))
 (segment (start 132.08 104.14) (end 132.08 104.14) (width 0.25) (layer F.Cu) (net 23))
 (via (at 132.08 104.14) (size 0.8) (drill 0.4) (layers F.Cu B.Cu) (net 23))
 (segment (start 106.68 124.46) (end 106.68 129.54) (width 0.25) (layer B.Cu) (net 14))
 (segment (start 144.78 96.52) (end 144.78 129.54) (width 0.25) (layer B.Cu) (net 14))
 (segment (start 144.78 86.36) (end 144.78 96.52) (width 0.25) (layer B.Cu) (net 14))
 (segment (start 106.68 129.54) (end 106.68 129.54) (width 0.25) (layer B.Cu) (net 14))
 (via (at 106.68 129.54) (size 0.8) (drill 0.4) (layers F.Cu B.Cu) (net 14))
 (segment (start 144.78 129.54) (end 144.78 129.54) (width 0.25) (layer B.Cu) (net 14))
 (via (at 144.78 129.54) (size 0.8) (drill 0.4) (layers F.Cu B.Cu) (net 14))
 (segment (start 144.78 129.54) (end 106.68 129.54) (width 0.25) (layer F.Cu) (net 14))
 (segment (start 142.24 86.36) (end 142.24 91.44) (width 0.25) (layer B.Cu) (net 16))
 (segment (start 104.14 109.22) (end 104.14 99.06) (width 0.25) (layer B.Cu) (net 16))
 (segment (start 142.24 91.44) (end 142.24 99.06) (width 0.25) (layer B.Cu) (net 16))
 (segment (start 104.14 99.06) (end 104.14 99.06) (width 0.25) (layer B.Cu) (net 16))
 (via (at 104.14 99.06) (size 0.8) (drill 0.4) (layers F.Cu B.Cu) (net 16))
 (segment (start 142.24 99.06) (end 142.24 99.06) (width 0.25) (layer B.Cu) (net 16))
 (via (at 142.24 99.06) (size 0.8) (drill 0.4) (layers F.Cu B.Cu) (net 16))
 (segment (start 104.14 99.06) (end 142.24 99.06) (width 0.25) (layer F.Cu) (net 16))
 (segment (start 101.6 101.6) (end 101.6 91.44) (width 0.25) (layer B.Cu) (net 8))
 (segment (start 101.6 109.22) (end 101.6 101.6) (width 0.25) (layer B.Cu) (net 8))
 (segment (start 154.94 86.36) (end 154.94 91.44) (width 0.25) (layer B.Cu) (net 8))
 (segment (start 101.6 91.44) (end 101.6 91.44) (width 0.25) (layer B.Cu) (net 8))
 (via (at 101.6 91.44) (size 0.8) (drill 0.4) (layers F.Cu B.Cu) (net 8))
 (segment (start 154.94 91.44) (end 154.94 91.44) (width 0.25) (layer B.Cu) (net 8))
 (via (at 154.94 91.44) (size 0.8) (drill 0.4) (layers F.Cu B.Cu) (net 8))
 (segment (start 154.94 91.44) (end 101.6 91.44) (width 0.25) (layer F.Cu) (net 8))
 (segment (start 132.08 86.36) (end 132.08 91.44) (width 0.25) (layer B.Cu) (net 23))
 (segment (start 132.08 91.44) (end 132.08 104.14) (width 0.25) (layer B.Cu) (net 23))
 (segment (start 93.98 109.22) (end 93.98 104.14) (width 0.25) (layer B.Cu) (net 23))
 (segment (start 93.98 104.14) (end 93.98 104.14) (width 0.25) (layer B.Cu) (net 23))
 (via (at 93.98 104.14) (size 0.8) (drill 0.4) (layers F.Cu B.Cu) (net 23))
 (segment (start 93.98 104.14) (end 93.98 104.14) (width 0.25) (layer B.Cu) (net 23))
 (via (at 93.98 104.14) (size 0.8) (drill 0.4) (layers F.Cu B.Cu) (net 23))
 (segment (start 134.62 86.36) (end 134.62 91.44) (width 0.25) (layer B.Cu) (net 21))
 (segment (start 134.62 91.44) (end 134.62 104.14) (width 0.25) (layer B.Cu) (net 21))
 (segment (start 177.8 109.22) (end 177.8 104.14) (width 0.25) (layer B.Cu) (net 21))
 (segment (start 177.8 104.14) (end 177.8 104.14) (width 0.25) (layer B.Cu) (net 21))
 (via (at 177.8 104.14) (size 0.8) (drill 0.4) (layers F.Cu B.Cu) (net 21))
 (segment (start 177.8 104.14) (end 134.62 104.14) (width 0.25) (layer F.Cu) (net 21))
 (segment (start 134.62 104.14) (end 134.62 104.14) (width 0.25) (layer F.Cu) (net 21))
 (via (at 134.62 104.14) (size 0.8) (drill 0.4) (layers F.Cu B.Cu) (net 21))
 (segment (start 185.42 109.22) (end 185.42 101.6) (width 0.25) (layer B.Cu) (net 10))
 (segment (start 152.4 91.44) (end 152.4 99.06) (width 0.25) (layer B.Cu) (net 10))
 (segment (start 152.4 86.36) (end 152.4 91.44) (width 0.25) (layer B.Cu) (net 10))
 (segment (start 185.42 101.6) (end 185.42 99.06) (width 0.25) (layer B.Cu) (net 10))
 (segment (start 152.4 99.06) (end 152.4 99.06) (width 0.25) (layer B.Cu) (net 10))
 (via (at 152.4 99.06) (size 0.8) (drill 0.4) (layers F.Cu B.Cu) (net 10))
 (segment (start 185.42 99.06) (end 185.42 99.06) (width 0.25) (layer B.Cu) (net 10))
 (via (at 185.42 99.06) (size 0.8) (drill 0.4) (layers F.Cu B.Cu) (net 10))
 (segment (start 152.4 99.06) (end 185.42 99.06) (width 0.25) (layer F.Cu) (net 10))
 (segment (start 139.7 86.36) (end 139.7 91.44) (width 0.25) (layer B.Cu) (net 18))
 (segment (start 139.7 91.44) (end 139.7 101.6) (width 0.25) (layer B.Cu) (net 18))
 (segment (start 187.96 109.22) (end 187.96 104.14) (width 0.25) (layer B.Cu) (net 18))
 (segment (start 187.96 104.14) (end 187.96 101.6) (width 0.25) (layer B.Cu) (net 18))
 (segment (start 139.7 101.6) (end 139.7 101.6) (width 0.25) (layer B.Cu) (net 18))
 (via (at 139.7 101.6) (size 0.8) (drill 0.4) (layers F.Cu B.Cu) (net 18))
 (segment (start 187.96 101.6) (end 187.96 101.6) (width 0.25) (layer B.Cu) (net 18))
 (via (at 187.96 101.6) (size 0.8) (drill 0.4) (layers F.Cu B.Cu) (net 18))
 (segment (start 187.96 101.6) (end 139.7 101.6) (width 0.25) (layer F.Cu) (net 18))
 (segment (start 147.32 93.98) (end 147.32 129.54) (width 0.25) (layer B.Cu) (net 13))
 (segment (start 147.32 86.36) (end 147.32 93.98) (width 0.25) (layer B.Cu) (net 13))
 (segment (start 190.5 124.46) (end 190.5 129.54) (width 0.25) (layer B.Cu) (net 13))
 (segment (start 147.32 129.54) (end 147.32 129.54) (width 0.25) (layer B.Cu) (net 13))
 (via (at 147.32 129.54) (size 0.8) (drill 0.4) (layers F.Cu B.Cu) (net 13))
 (segment (start 190.5 129.54) (end 190.5 129.54) (width 0.25) (layer B.Cu) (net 13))
 (via (at 190.5 129.54) (size 0.8) (drill 0.4) (layers F.Cu B.Cu) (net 13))
 (segment (start 190.5 129.54) (end 147.32 129.54) (width 0.25) (layer F.Cu) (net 13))
 (via (at 137.16 93.98) (size 0.8) (drill 0.4) (layers F.Cu B.Cu) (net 1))
 (segment (start 137.16 86.36) (end 137.16 93.98) (width 0.25) (layer B.Cu) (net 1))
 (segment (start 137.16 93.98) (end 149.86 93.98) (width 0.25) (layer F.Cu) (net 1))
 (via (at 149.86 93.98) (size 0.8) (drill 0.4) (layers F.Cu B.Cu) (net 1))
 (segment (start 149.86 86.36) (end 149.86 93.98) (width 0.25) (layer B.Cu) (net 1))
 (segment (start 149.86 93.98) (end 182.88 93.98) (width 0.25) (layer F.Cu) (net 1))
 (via (at 182.88 93.98) (size 0.8) (drill 0.4) (layers F.Cu B.Cu) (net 1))
 (segment (start 182.88 83.82) (end 182.88 93.98) (width 0.25) (layer B.Cu) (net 1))
 (segment (start 180.34 83.82) (end 180.34 88.9) (width 0.25) (layer B.Cu) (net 2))
 (via (at 180.34 60.96) (size 0.8) (drill 0.4) (layers F.Cu B.Cu) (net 2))
 (segment (start 180.34 83.82) (end 180.34 60.96) (width 0.25) (layer B.Cu) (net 2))
 (via (at 142.24 60.96) (size 0.8) (drill 0.4) (layers F.Cu B.Cu) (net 2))
 (segment (start 180.34 60.96) (end 142.24 60.96) (width 0.25) (layer F.Cu) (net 2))
 (segment (start 142.24 60.96) (end 142.24 78.74) (width 0.25) (layer B.Cu) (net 2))
 (segment (start 129.54 86.36) (end 129.54 96.52) (width 0.25) (layer B.Cu) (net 3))
 (via (at 129.54 96.52) (size 0.8) (drill 0.4) (layers F.Cu B.Cu) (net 3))
 (segment (start 129.54 96.52) (end 177.8 96.52) (width 0.25) (layer F.Cu) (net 3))
 (via (at 177.8 96.52) (size 0.8) (drill 0.4) (layers F.Cu B.Cu) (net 3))
 (segment (start 177.8 83.82) (end 177.8 96.52) (width 0.25) (layer B.Cu) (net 3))
 (segment (start 157.48 78.74) (end 157.48 63.5) (width 0.25) (layer B.Cu) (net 4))
 (segment (start 157.48 63.5) (end 157.48 63.5) (width 0.25) (layer B.Cu) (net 4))
 (via (at 157.48 63.5) (size 0.8) (drill 0.4) (layers F.Cu B.Cu) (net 4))
 (via (at 175.26 63.5) (size 0.8) (drill 0.4) (layers F.Cu B.Cu) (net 4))
 (segment (start 157.48 63.5) (end 175.26 63.5) (width 0.25) (layer F.Cu) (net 4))
 (segment (start 175.26 63.5) (end 175.26 83.82) (width 0.25) (layer B.Cu) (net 4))
 (via (at 157.48 91.44) (size 0.8) (drill 0.4) (layers F.Cu B.Cu) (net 5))
 (segment (start 157.48 86.36) (end 157.48 91.44) (width 0.25) (layer B.Cu) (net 5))
 (segment (start 157.48 91.44) (end 172.72 91.44) (width 0.25) (layer F.Cu) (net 5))
 (via (at 172.72 91.44) (size 0.8) (drill 0.4) (layers F.Cu B.Cu) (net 5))
 (segment (start 172.72 83.82) (end 172.72 91.44) (width 0.25) (layer B.Cu) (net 5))
 (segment (start 144.78 63.5) (end 144.78 63.5) (width 0.25) (layer B.Cu) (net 15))
 (segment (start 144.78 78.74) (end 144.78 58.42) (width 0.25) (layer B.Cu) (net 15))
 (via (at 144.78 58.42) (size 0.8) (drill 0.4) (layers F.Cu B.Cu) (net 15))
 (via (at 165.1 58.42) (size 0.8) (drill 0.4) (layers F.Cu B.Cu) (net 15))
 (segment (start 144.78 58.42) (end 165.1 58.42) (width 0.25) (layer F.Cu) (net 15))
 (segment (start 165.1 58.42) (end 165.1 88.9) (width 0.25) (layer B.Cu) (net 15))
 (via (at 165.1 88.9) (size 0.8) (drill 0.4) (layers F.Cu B.Cu) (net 15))
 (segment (start 165.1 88.9) (end 175.26 88.9) (width 0.25) (layer F.Cu) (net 15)))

